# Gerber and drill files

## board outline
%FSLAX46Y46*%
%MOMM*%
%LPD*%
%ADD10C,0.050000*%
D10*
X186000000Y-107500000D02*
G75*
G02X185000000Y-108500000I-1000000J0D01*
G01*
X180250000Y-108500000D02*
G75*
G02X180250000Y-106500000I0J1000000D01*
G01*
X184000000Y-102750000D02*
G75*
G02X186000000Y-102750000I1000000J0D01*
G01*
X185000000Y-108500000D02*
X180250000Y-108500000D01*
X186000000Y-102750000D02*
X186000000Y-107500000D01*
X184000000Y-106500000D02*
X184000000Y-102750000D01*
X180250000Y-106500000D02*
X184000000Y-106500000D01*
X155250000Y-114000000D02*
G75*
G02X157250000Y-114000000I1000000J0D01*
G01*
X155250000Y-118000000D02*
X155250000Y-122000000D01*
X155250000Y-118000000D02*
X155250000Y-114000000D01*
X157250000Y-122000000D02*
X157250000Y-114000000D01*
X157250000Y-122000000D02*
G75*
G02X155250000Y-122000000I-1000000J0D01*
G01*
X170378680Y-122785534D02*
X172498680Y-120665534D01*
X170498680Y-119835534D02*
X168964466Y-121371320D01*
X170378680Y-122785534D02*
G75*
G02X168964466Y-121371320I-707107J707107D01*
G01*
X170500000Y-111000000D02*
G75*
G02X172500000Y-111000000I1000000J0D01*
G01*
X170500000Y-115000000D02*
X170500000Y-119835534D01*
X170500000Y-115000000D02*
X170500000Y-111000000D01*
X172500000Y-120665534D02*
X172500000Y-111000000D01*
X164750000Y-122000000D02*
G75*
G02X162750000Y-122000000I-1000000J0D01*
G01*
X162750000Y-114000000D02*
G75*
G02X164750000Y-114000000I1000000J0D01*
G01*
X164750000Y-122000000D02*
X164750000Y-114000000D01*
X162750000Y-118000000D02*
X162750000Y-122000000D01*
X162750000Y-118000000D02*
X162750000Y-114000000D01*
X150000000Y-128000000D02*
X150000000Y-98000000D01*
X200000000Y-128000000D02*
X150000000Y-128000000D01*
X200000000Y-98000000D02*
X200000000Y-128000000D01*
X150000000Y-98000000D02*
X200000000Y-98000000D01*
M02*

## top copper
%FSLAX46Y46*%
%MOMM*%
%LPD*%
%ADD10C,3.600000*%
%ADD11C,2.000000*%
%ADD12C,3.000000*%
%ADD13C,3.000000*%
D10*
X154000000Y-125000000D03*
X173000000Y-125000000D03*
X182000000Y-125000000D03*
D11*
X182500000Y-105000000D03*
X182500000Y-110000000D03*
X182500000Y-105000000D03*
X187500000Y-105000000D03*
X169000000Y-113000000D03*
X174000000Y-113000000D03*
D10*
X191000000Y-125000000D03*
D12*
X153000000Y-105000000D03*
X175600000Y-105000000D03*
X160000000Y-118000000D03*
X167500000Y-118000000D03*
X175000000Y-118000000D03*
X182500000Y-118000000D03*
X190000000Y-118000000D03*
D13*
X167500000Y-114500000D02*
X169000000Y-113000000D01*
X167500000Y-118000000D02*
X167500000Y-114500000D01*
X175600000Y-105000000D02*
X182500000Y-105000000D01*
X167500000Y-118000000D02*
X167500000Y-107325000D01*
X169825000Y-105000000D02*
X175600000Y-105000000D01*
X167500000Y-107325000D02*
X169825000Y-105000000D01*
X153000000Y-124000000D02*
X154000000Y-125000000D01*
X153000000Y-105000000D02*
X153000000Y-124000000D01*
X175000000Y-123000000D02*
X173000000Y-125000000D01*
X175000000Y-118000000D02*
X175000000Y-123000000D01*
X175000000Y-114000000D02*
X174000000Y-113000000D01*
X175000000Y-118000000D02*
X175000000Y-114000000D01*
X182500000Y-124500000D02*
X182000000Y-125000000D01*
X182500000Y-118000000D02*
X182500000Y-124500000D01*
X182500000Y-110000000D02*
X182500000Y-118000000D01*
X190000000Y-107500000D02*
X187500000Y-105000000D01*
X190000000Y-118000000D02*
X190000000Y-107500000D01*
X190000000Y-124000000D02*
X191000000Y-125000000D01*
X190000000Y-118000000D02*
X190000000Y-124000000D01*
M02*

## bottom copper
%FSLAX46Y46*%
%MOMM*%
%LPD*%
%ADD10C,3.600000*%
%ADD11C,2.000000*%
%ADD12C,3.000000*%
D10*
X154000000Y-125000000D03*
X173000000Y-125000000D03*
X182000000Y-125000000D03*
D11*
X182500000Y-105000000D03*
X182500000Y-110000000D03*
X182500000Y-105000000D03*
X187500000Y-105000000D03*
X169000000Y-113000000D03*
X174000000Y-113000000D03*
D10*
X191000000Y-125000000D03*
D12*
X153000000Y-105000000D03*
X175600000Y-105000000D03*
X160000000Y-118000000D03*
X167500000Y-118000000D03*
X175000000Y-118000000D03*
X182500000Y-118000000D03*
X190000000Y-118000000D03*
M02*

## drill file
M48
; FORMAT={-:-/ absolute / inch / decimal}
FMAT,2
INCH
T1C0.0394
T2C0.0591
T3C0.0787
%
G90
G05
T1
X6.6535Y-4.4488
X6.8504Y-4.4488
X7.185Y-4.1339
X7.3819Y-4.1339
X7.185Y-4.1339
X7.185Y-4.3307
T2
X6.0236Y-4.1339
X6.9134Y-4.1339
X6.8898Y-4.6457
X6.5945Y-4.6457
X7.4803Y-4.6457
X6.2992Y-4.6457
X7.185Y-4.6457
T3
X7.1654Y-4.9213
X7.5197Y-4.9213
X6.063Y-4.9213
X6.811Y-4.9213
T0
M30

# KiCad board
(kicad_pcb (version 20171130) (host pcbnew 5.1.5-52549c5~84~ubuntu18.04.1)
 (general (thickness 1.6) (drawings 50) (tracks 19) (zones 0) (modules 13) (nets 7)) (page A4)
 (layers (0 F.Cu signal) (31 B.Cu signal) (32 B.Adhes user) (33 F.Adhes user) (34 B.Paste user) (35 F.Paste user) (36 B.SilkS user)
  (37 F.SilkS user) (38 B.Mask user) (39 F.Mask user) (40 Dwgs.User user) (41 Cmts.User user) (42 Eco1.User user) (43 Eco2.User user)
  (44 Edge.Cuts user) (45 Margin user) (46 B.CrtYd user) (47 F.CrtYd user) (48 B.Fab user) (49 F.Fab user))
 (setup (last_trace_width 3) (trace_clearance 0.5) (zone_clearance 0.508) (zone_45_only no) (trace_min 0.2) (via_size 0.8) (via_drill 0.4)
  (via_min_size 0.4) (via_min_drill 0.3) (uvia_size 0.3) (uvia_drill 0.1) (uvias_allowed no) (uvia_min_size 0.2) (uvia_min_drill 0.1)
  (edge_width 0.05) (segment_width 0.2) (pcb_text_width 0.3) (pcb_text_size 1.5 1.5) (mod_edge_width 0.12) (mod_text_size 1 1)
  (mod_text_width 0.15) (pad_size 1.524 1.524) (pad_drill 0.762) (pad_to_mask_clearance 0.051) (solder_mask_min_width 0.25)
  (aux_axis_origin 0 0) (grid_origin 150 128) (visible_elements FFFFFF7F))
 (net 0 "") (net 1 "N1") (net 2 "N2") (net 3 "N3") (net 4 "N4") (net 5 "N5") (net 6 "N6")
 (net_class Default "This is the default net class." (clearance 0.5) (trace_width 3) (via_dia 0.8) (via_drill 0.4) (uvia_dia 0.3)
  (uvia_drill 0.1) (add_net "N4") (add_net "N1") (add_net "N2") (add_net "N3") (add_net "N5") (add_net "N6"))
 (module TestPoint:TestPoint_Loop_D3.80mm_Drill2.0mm (layer F.Cu) (at 154 125)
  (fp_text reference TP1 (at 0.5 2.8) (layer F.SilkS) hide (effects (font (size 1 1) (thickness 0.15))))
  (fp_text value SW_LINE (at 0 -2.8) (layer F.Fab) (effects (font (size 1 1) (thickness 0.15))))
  (pad 1 thru_hole circle (at 0 0) (size 3.6 3.6) (drill 2) (layers *.Cu *.Mask) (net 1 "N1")))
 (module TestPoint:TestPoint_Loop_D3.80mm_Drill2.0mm (layer F.Cu) (at 173 125)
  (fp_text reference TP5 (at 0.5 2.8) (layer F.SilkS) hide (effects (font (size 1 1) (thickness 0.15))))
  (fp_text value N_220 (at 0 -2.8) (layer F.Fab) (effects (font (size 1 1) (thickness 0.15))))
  (pad 1 thru_hole circle (at 0 0) (size 3.6 3.6) (drill 2) (layers *.Cu *.Mask) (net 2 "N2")))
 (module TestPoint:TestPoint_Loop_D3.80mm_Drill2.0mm (layer F.Cu) (at 182 125)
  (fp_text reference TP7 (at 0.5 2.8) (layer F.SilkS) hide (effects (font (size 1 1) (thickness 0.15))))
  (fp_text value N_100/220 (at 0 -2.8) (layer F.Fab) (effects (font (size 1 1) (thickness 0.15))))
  (pad 1 thru_hole circle (at 0 0) (size 3.6 3.6) (drill 2) (layers *.Cu *.Mask) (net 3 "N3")))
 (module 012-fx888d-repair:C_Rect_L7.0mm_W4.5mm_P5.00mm (layer F.Cu) (at 182.5 105 270)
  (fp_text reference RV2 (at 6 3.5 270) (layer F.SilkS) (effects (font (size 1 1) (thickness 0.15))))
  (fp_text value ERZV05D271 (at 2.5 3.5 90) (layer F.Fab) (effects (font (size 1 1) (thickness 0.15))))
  (pad 1 thru_hole circle (at 0 0 270) (size 2 2) (drill 1) (layers *.Cu *.Mask) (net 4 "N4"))
  (pad 2 thru_hole circle (at 5 0 270) (size 2 2) (drill 1) (layers *.Cu *.Mask) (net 3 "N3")))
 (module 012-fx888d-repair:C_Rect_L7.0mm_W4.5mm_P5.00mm (layer F.Cu) (at 182.5 105)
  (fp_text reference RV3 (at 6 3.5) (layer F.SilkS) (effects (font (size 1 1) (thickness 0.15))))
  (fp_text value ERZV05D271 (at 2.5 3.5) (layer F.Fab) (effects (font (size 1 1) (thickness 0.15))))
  (pad 1 thru_hole circle (at 0 0) (size 2 2) (drill 1) (layers *.Cu *.Mask) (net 4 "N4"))
  (pad 2 thru_hole circle (at 5 0) (size 2 2) (drill 1) (layers *.Cu *.Mask) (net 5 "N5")))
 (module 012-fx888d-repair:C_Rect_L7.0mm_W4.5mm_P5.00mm (layer F.Cu) (at 169 113)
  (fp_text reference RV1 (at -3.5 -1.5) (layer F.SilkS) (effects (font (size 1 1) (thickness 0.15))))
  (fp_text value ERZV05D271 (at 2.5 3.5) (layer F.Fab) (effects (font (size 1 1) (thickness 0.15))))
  (pad 1 thru_hole circle (at 0 0) (size 2 2) (drill 1) (layers *.Cu *.Mask) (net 4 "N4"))
  (pad 2 thru_hole circle (at 5 0) (size 2 2) (drill 1) (layers *.Cu *.Mask) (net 2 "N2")))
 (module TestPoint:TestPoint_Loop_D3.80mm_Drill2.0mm (layer F.Cu) (at 191 125)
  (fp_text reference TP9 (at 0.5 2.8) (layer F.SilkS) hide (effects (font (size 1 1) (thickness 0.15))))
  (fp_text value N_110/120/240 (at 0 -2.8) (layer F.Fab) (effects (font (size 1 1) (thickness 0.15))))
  (pad 1 thru_hole circle (at 0 0) (size 3.6 3.6) (drill 2) (layers *.Cu *.Mask) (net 5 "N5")))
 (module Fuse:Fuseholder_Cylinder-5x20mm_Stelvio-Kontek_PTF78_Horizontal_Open (layer F.Cu) (at 175.6 105 180)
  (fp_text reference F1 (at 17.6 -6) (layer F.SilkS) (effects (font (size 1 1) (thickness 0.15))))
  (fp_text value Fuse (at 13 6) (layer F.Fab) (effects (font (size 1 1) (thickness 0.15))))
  (pad 2 thru_hole circle (at 22.6 0 180) (size 3 3) (drill 1.5) (layers *.Cu *.Mask) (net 1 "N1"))
  (pad 1 thru_hole circle (at 0 0 180) (size 3 3) (drill 1.5) (layers *.Cu *.Mask) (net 4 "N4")))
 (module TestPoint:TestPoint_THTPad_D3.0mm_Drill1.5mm (layer F.Cu) (at 160 118)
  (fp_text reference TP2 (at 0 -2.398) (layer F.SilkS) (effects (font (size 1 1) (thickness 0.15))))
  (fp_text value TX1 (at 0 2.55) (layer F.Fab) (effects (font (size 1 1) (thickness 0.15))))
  (pad 1 thru_hole circle (at 0 0) (size 3 3) (drill 1.5) (layers *.Cu *.Mask) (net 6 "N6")))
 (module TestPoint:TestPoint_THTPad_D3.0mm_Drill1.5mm (layer F.Cu) (at 167.5 118)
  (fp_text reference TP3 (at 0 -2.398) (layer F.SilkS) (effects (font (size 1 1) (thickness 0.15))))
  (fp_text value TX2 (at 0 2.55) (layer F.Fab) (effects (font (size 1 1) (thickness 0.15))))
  (pad 1 thru_hole circle (at 0 0) (size 3 3) (drill 1.5) (layers *.Cu *.Mask) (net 4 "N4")))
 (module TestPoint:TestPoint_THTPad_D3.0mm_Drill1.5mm (layer F.Cu) (at 175 118)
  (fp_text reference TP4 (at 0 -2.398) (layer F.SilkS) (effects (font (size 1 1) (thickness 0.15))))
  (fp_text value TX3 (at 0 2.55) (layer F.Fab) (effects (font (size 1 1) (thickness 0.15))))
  (pad 1 thru_hole circle (at 0 0) (size 3 3) (drill 1.5) (layers *.Cu *.Mask) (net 2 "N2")))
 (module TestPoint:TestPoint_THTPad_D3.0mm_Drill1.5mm (layer F.Cu) (at 182.5 118)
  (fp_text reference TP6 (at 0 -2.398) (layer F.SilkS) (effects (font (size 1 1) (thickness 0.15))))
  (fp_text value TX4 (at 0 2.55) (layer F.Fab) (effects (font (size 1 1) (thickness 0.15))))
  (pad 1 thru_hole circle (at 0 0) (size 3 3) (drill 1.5) (layers *.Cu *.Mask) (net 3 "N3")))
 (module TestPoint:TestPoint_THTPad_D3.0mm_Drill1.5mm (layer F.Cu) (at 190 118)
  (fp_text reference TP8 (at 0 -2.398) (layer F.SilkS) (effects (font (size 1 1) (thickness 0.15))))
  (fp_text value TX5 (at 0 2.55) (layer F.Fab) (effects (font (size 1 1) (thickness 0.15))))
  (pad 1 thru_hole circle (at 0 0) (size 3 3) (drill 1.5) (layers *.Cu *.Mask) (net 5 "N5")))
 (gr_arc (start 185 107.5) (end 185 108.5) (angle -90) (layer Edge.Cuts) (width 0.05))
 (gr_arc (start 180.25 107.5) (end 180.25 106.5) (angle -180) (layer Edge.Cuts) (width 0.05))
 (gr_arc (start 185 102.75) (end 186 102.75) (angle -180) (layer Edge.Cuts) (width 0.05))
 (gr_line (start 185 108.5) (end 180.25 108.5) (layer Edge.Cuts) (width 0.05))
 (gr_line (start 186 102.75) (end 186 107.5) (layer Edge.Cuts) (width 0.05))
 (gr_line (start 184 106.5) (end 184 102.75) (layer Edge.Cuts) (width 0.05))
 (gr_line (start 180.25 106.5) (end 184 106.5) (layer Edge.Cuts) (width 0.05))
 (gr_arc (start 156.25 114) (end 157.25 114) (angle -180) (layer Edge.Cuts) (width 0.05))
 (gr_line (start 155.25 118) (end 155.25 122) (layer Edge.Cuts) (width 0.05))
 (gr_line (start 155.25 118) (end 155.25 114) (layer Edge.Cuts) (width 0.05))
 (gr_line (start 157.25 122) (end 157.25 114) (layer Edge.Cuts) (width 0.05))
 (gr_arc (start 156.25 122) (end 155.25 122) (angle -180) (layer Edge.Cuts) (width 0.05))
 (gr_line (start 170.37868 122.785534) (end 172.49868 120.665534) (layer Edge.Cuts) (width 0.05))
 (gr_line (start 170.49868 119.835534) (end 168.964466 121.37132) (layer Edge.Cuts) (width 0.05))
 (gr_arc (start 169.671573 122.078427) (end 168.964466 121.37132) (angle -180) (layer Edge.Cuts) (width 0.05))
 (gr_arc (start 171.5 111) (end 172.5 111) (angle -180) (layer Edge.Cuts) (width 0.05))
 (gr_line (start 170.5 115) (end 170.5 119.835534) (layer Edge.Cuts) (width 0.05))
 (gr_line (start 170.5 115) (end 170.5 111) (layer Edge.Cuts) (width 0.05))
 (gr_line (start 172.5 120.665534) (end 172.5 111) (layer Edge.Cuts) (width 0.05))
 (gr_arc (start 163.75 122) (end 162.75 122) (angle -180) (layer Edge.Cuts) (width 0.05))
 (gr_arc (start 163.75 114) (end 164.75 114) (angle -180) (layer Edge.Cuts) (width 0.05))
 (gr_line (start 164.75 122) (end 164.75 114) (layer Edge.Cuts) (width 0.05))
 (gr_line (start 162.75 118) (end 162.75 122) (layer Edge.Cuts) (width 0.05))
 (gr_line (start 162.75 118) (end 162.75 114) (layer Edge.Cuts) (width 0.05))
 (gr_line (start 150 128) (end 150 98) (layer Edge.Cuts) (width 0.05))
 (gr_line (start 200 128) (end 150 128) (layer Edge.Cuts) (width 0.05))
 (gr_line (start 200 98) (end 200 128) (layer Edge.Cuts) (width 0.05))
 (gr_line (start 150 98) (end 200 98) (layer Edge.Cuts) (width 0.05))
 (segment (start 167.5 114.5) (end 169 113) (width 3) (layer F.Cu) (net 4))
 (segment (start 167.5 118) (end 167.5 114.5) (width 3) (layer F.Cu) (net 4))
 (segment (start 175.6 105) (end 182.5 105) (width 3) (layer F.Cu) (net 4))
 (segment (start 167.5 118) (end 167.5 107.325) (width 3) (layer F.Cu) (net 4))
 (segment (start 169.825 105) (end 175.6 105) (width 3) (layer F.Cu) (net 4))
 (segment (start 167.5 107.325) (end 169.825 105) (width 3) (layer F.Cu) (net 4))
 (segment (start 153 124) (end 154 125) (width 3) (layer F.Cu) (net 1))
 (segment (start 153 105) (end 153 124) (width 3) (layer F.Cu) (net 1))
 (segment (start 175 123) (end 173 125) (width 3) (layer F.Cu) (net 2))
 (segment (start 175 118) (end 175 123) (width 3) (layer F.Cu) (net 2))
 (segment (start 175 114) (end 174 113) (width 3) (layer F.Cu) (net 2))
 (segment (start 175 118) (end 175 114) (width 3) (layer F.Cu) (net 2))
 (segment (start 182.5 124.5) (end 182 125) (width 3) (layer F.Cu) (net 3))
 (segment (start 182.5 118) (end 182.5 124.5) (width 3) (layer F.Cu) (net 3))
 (segment (start 182.5 110) (end 182.5 118) (width 3) (layer F.Cu) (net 3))
 (segment (start 190 107.5) (end 187.5 105) (width 3) (layer F.Cu) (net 5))
 (segment (start 190 118) (end 190 107.5) (width 3) (layer F.Cu) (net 5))
 (segment (start 190 124) (end 191 125) (width 3) (layer F.Cu) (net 5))
 (segment (start 190 118) (end 190 124) (width 3) (layer F.Cu) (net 5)))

